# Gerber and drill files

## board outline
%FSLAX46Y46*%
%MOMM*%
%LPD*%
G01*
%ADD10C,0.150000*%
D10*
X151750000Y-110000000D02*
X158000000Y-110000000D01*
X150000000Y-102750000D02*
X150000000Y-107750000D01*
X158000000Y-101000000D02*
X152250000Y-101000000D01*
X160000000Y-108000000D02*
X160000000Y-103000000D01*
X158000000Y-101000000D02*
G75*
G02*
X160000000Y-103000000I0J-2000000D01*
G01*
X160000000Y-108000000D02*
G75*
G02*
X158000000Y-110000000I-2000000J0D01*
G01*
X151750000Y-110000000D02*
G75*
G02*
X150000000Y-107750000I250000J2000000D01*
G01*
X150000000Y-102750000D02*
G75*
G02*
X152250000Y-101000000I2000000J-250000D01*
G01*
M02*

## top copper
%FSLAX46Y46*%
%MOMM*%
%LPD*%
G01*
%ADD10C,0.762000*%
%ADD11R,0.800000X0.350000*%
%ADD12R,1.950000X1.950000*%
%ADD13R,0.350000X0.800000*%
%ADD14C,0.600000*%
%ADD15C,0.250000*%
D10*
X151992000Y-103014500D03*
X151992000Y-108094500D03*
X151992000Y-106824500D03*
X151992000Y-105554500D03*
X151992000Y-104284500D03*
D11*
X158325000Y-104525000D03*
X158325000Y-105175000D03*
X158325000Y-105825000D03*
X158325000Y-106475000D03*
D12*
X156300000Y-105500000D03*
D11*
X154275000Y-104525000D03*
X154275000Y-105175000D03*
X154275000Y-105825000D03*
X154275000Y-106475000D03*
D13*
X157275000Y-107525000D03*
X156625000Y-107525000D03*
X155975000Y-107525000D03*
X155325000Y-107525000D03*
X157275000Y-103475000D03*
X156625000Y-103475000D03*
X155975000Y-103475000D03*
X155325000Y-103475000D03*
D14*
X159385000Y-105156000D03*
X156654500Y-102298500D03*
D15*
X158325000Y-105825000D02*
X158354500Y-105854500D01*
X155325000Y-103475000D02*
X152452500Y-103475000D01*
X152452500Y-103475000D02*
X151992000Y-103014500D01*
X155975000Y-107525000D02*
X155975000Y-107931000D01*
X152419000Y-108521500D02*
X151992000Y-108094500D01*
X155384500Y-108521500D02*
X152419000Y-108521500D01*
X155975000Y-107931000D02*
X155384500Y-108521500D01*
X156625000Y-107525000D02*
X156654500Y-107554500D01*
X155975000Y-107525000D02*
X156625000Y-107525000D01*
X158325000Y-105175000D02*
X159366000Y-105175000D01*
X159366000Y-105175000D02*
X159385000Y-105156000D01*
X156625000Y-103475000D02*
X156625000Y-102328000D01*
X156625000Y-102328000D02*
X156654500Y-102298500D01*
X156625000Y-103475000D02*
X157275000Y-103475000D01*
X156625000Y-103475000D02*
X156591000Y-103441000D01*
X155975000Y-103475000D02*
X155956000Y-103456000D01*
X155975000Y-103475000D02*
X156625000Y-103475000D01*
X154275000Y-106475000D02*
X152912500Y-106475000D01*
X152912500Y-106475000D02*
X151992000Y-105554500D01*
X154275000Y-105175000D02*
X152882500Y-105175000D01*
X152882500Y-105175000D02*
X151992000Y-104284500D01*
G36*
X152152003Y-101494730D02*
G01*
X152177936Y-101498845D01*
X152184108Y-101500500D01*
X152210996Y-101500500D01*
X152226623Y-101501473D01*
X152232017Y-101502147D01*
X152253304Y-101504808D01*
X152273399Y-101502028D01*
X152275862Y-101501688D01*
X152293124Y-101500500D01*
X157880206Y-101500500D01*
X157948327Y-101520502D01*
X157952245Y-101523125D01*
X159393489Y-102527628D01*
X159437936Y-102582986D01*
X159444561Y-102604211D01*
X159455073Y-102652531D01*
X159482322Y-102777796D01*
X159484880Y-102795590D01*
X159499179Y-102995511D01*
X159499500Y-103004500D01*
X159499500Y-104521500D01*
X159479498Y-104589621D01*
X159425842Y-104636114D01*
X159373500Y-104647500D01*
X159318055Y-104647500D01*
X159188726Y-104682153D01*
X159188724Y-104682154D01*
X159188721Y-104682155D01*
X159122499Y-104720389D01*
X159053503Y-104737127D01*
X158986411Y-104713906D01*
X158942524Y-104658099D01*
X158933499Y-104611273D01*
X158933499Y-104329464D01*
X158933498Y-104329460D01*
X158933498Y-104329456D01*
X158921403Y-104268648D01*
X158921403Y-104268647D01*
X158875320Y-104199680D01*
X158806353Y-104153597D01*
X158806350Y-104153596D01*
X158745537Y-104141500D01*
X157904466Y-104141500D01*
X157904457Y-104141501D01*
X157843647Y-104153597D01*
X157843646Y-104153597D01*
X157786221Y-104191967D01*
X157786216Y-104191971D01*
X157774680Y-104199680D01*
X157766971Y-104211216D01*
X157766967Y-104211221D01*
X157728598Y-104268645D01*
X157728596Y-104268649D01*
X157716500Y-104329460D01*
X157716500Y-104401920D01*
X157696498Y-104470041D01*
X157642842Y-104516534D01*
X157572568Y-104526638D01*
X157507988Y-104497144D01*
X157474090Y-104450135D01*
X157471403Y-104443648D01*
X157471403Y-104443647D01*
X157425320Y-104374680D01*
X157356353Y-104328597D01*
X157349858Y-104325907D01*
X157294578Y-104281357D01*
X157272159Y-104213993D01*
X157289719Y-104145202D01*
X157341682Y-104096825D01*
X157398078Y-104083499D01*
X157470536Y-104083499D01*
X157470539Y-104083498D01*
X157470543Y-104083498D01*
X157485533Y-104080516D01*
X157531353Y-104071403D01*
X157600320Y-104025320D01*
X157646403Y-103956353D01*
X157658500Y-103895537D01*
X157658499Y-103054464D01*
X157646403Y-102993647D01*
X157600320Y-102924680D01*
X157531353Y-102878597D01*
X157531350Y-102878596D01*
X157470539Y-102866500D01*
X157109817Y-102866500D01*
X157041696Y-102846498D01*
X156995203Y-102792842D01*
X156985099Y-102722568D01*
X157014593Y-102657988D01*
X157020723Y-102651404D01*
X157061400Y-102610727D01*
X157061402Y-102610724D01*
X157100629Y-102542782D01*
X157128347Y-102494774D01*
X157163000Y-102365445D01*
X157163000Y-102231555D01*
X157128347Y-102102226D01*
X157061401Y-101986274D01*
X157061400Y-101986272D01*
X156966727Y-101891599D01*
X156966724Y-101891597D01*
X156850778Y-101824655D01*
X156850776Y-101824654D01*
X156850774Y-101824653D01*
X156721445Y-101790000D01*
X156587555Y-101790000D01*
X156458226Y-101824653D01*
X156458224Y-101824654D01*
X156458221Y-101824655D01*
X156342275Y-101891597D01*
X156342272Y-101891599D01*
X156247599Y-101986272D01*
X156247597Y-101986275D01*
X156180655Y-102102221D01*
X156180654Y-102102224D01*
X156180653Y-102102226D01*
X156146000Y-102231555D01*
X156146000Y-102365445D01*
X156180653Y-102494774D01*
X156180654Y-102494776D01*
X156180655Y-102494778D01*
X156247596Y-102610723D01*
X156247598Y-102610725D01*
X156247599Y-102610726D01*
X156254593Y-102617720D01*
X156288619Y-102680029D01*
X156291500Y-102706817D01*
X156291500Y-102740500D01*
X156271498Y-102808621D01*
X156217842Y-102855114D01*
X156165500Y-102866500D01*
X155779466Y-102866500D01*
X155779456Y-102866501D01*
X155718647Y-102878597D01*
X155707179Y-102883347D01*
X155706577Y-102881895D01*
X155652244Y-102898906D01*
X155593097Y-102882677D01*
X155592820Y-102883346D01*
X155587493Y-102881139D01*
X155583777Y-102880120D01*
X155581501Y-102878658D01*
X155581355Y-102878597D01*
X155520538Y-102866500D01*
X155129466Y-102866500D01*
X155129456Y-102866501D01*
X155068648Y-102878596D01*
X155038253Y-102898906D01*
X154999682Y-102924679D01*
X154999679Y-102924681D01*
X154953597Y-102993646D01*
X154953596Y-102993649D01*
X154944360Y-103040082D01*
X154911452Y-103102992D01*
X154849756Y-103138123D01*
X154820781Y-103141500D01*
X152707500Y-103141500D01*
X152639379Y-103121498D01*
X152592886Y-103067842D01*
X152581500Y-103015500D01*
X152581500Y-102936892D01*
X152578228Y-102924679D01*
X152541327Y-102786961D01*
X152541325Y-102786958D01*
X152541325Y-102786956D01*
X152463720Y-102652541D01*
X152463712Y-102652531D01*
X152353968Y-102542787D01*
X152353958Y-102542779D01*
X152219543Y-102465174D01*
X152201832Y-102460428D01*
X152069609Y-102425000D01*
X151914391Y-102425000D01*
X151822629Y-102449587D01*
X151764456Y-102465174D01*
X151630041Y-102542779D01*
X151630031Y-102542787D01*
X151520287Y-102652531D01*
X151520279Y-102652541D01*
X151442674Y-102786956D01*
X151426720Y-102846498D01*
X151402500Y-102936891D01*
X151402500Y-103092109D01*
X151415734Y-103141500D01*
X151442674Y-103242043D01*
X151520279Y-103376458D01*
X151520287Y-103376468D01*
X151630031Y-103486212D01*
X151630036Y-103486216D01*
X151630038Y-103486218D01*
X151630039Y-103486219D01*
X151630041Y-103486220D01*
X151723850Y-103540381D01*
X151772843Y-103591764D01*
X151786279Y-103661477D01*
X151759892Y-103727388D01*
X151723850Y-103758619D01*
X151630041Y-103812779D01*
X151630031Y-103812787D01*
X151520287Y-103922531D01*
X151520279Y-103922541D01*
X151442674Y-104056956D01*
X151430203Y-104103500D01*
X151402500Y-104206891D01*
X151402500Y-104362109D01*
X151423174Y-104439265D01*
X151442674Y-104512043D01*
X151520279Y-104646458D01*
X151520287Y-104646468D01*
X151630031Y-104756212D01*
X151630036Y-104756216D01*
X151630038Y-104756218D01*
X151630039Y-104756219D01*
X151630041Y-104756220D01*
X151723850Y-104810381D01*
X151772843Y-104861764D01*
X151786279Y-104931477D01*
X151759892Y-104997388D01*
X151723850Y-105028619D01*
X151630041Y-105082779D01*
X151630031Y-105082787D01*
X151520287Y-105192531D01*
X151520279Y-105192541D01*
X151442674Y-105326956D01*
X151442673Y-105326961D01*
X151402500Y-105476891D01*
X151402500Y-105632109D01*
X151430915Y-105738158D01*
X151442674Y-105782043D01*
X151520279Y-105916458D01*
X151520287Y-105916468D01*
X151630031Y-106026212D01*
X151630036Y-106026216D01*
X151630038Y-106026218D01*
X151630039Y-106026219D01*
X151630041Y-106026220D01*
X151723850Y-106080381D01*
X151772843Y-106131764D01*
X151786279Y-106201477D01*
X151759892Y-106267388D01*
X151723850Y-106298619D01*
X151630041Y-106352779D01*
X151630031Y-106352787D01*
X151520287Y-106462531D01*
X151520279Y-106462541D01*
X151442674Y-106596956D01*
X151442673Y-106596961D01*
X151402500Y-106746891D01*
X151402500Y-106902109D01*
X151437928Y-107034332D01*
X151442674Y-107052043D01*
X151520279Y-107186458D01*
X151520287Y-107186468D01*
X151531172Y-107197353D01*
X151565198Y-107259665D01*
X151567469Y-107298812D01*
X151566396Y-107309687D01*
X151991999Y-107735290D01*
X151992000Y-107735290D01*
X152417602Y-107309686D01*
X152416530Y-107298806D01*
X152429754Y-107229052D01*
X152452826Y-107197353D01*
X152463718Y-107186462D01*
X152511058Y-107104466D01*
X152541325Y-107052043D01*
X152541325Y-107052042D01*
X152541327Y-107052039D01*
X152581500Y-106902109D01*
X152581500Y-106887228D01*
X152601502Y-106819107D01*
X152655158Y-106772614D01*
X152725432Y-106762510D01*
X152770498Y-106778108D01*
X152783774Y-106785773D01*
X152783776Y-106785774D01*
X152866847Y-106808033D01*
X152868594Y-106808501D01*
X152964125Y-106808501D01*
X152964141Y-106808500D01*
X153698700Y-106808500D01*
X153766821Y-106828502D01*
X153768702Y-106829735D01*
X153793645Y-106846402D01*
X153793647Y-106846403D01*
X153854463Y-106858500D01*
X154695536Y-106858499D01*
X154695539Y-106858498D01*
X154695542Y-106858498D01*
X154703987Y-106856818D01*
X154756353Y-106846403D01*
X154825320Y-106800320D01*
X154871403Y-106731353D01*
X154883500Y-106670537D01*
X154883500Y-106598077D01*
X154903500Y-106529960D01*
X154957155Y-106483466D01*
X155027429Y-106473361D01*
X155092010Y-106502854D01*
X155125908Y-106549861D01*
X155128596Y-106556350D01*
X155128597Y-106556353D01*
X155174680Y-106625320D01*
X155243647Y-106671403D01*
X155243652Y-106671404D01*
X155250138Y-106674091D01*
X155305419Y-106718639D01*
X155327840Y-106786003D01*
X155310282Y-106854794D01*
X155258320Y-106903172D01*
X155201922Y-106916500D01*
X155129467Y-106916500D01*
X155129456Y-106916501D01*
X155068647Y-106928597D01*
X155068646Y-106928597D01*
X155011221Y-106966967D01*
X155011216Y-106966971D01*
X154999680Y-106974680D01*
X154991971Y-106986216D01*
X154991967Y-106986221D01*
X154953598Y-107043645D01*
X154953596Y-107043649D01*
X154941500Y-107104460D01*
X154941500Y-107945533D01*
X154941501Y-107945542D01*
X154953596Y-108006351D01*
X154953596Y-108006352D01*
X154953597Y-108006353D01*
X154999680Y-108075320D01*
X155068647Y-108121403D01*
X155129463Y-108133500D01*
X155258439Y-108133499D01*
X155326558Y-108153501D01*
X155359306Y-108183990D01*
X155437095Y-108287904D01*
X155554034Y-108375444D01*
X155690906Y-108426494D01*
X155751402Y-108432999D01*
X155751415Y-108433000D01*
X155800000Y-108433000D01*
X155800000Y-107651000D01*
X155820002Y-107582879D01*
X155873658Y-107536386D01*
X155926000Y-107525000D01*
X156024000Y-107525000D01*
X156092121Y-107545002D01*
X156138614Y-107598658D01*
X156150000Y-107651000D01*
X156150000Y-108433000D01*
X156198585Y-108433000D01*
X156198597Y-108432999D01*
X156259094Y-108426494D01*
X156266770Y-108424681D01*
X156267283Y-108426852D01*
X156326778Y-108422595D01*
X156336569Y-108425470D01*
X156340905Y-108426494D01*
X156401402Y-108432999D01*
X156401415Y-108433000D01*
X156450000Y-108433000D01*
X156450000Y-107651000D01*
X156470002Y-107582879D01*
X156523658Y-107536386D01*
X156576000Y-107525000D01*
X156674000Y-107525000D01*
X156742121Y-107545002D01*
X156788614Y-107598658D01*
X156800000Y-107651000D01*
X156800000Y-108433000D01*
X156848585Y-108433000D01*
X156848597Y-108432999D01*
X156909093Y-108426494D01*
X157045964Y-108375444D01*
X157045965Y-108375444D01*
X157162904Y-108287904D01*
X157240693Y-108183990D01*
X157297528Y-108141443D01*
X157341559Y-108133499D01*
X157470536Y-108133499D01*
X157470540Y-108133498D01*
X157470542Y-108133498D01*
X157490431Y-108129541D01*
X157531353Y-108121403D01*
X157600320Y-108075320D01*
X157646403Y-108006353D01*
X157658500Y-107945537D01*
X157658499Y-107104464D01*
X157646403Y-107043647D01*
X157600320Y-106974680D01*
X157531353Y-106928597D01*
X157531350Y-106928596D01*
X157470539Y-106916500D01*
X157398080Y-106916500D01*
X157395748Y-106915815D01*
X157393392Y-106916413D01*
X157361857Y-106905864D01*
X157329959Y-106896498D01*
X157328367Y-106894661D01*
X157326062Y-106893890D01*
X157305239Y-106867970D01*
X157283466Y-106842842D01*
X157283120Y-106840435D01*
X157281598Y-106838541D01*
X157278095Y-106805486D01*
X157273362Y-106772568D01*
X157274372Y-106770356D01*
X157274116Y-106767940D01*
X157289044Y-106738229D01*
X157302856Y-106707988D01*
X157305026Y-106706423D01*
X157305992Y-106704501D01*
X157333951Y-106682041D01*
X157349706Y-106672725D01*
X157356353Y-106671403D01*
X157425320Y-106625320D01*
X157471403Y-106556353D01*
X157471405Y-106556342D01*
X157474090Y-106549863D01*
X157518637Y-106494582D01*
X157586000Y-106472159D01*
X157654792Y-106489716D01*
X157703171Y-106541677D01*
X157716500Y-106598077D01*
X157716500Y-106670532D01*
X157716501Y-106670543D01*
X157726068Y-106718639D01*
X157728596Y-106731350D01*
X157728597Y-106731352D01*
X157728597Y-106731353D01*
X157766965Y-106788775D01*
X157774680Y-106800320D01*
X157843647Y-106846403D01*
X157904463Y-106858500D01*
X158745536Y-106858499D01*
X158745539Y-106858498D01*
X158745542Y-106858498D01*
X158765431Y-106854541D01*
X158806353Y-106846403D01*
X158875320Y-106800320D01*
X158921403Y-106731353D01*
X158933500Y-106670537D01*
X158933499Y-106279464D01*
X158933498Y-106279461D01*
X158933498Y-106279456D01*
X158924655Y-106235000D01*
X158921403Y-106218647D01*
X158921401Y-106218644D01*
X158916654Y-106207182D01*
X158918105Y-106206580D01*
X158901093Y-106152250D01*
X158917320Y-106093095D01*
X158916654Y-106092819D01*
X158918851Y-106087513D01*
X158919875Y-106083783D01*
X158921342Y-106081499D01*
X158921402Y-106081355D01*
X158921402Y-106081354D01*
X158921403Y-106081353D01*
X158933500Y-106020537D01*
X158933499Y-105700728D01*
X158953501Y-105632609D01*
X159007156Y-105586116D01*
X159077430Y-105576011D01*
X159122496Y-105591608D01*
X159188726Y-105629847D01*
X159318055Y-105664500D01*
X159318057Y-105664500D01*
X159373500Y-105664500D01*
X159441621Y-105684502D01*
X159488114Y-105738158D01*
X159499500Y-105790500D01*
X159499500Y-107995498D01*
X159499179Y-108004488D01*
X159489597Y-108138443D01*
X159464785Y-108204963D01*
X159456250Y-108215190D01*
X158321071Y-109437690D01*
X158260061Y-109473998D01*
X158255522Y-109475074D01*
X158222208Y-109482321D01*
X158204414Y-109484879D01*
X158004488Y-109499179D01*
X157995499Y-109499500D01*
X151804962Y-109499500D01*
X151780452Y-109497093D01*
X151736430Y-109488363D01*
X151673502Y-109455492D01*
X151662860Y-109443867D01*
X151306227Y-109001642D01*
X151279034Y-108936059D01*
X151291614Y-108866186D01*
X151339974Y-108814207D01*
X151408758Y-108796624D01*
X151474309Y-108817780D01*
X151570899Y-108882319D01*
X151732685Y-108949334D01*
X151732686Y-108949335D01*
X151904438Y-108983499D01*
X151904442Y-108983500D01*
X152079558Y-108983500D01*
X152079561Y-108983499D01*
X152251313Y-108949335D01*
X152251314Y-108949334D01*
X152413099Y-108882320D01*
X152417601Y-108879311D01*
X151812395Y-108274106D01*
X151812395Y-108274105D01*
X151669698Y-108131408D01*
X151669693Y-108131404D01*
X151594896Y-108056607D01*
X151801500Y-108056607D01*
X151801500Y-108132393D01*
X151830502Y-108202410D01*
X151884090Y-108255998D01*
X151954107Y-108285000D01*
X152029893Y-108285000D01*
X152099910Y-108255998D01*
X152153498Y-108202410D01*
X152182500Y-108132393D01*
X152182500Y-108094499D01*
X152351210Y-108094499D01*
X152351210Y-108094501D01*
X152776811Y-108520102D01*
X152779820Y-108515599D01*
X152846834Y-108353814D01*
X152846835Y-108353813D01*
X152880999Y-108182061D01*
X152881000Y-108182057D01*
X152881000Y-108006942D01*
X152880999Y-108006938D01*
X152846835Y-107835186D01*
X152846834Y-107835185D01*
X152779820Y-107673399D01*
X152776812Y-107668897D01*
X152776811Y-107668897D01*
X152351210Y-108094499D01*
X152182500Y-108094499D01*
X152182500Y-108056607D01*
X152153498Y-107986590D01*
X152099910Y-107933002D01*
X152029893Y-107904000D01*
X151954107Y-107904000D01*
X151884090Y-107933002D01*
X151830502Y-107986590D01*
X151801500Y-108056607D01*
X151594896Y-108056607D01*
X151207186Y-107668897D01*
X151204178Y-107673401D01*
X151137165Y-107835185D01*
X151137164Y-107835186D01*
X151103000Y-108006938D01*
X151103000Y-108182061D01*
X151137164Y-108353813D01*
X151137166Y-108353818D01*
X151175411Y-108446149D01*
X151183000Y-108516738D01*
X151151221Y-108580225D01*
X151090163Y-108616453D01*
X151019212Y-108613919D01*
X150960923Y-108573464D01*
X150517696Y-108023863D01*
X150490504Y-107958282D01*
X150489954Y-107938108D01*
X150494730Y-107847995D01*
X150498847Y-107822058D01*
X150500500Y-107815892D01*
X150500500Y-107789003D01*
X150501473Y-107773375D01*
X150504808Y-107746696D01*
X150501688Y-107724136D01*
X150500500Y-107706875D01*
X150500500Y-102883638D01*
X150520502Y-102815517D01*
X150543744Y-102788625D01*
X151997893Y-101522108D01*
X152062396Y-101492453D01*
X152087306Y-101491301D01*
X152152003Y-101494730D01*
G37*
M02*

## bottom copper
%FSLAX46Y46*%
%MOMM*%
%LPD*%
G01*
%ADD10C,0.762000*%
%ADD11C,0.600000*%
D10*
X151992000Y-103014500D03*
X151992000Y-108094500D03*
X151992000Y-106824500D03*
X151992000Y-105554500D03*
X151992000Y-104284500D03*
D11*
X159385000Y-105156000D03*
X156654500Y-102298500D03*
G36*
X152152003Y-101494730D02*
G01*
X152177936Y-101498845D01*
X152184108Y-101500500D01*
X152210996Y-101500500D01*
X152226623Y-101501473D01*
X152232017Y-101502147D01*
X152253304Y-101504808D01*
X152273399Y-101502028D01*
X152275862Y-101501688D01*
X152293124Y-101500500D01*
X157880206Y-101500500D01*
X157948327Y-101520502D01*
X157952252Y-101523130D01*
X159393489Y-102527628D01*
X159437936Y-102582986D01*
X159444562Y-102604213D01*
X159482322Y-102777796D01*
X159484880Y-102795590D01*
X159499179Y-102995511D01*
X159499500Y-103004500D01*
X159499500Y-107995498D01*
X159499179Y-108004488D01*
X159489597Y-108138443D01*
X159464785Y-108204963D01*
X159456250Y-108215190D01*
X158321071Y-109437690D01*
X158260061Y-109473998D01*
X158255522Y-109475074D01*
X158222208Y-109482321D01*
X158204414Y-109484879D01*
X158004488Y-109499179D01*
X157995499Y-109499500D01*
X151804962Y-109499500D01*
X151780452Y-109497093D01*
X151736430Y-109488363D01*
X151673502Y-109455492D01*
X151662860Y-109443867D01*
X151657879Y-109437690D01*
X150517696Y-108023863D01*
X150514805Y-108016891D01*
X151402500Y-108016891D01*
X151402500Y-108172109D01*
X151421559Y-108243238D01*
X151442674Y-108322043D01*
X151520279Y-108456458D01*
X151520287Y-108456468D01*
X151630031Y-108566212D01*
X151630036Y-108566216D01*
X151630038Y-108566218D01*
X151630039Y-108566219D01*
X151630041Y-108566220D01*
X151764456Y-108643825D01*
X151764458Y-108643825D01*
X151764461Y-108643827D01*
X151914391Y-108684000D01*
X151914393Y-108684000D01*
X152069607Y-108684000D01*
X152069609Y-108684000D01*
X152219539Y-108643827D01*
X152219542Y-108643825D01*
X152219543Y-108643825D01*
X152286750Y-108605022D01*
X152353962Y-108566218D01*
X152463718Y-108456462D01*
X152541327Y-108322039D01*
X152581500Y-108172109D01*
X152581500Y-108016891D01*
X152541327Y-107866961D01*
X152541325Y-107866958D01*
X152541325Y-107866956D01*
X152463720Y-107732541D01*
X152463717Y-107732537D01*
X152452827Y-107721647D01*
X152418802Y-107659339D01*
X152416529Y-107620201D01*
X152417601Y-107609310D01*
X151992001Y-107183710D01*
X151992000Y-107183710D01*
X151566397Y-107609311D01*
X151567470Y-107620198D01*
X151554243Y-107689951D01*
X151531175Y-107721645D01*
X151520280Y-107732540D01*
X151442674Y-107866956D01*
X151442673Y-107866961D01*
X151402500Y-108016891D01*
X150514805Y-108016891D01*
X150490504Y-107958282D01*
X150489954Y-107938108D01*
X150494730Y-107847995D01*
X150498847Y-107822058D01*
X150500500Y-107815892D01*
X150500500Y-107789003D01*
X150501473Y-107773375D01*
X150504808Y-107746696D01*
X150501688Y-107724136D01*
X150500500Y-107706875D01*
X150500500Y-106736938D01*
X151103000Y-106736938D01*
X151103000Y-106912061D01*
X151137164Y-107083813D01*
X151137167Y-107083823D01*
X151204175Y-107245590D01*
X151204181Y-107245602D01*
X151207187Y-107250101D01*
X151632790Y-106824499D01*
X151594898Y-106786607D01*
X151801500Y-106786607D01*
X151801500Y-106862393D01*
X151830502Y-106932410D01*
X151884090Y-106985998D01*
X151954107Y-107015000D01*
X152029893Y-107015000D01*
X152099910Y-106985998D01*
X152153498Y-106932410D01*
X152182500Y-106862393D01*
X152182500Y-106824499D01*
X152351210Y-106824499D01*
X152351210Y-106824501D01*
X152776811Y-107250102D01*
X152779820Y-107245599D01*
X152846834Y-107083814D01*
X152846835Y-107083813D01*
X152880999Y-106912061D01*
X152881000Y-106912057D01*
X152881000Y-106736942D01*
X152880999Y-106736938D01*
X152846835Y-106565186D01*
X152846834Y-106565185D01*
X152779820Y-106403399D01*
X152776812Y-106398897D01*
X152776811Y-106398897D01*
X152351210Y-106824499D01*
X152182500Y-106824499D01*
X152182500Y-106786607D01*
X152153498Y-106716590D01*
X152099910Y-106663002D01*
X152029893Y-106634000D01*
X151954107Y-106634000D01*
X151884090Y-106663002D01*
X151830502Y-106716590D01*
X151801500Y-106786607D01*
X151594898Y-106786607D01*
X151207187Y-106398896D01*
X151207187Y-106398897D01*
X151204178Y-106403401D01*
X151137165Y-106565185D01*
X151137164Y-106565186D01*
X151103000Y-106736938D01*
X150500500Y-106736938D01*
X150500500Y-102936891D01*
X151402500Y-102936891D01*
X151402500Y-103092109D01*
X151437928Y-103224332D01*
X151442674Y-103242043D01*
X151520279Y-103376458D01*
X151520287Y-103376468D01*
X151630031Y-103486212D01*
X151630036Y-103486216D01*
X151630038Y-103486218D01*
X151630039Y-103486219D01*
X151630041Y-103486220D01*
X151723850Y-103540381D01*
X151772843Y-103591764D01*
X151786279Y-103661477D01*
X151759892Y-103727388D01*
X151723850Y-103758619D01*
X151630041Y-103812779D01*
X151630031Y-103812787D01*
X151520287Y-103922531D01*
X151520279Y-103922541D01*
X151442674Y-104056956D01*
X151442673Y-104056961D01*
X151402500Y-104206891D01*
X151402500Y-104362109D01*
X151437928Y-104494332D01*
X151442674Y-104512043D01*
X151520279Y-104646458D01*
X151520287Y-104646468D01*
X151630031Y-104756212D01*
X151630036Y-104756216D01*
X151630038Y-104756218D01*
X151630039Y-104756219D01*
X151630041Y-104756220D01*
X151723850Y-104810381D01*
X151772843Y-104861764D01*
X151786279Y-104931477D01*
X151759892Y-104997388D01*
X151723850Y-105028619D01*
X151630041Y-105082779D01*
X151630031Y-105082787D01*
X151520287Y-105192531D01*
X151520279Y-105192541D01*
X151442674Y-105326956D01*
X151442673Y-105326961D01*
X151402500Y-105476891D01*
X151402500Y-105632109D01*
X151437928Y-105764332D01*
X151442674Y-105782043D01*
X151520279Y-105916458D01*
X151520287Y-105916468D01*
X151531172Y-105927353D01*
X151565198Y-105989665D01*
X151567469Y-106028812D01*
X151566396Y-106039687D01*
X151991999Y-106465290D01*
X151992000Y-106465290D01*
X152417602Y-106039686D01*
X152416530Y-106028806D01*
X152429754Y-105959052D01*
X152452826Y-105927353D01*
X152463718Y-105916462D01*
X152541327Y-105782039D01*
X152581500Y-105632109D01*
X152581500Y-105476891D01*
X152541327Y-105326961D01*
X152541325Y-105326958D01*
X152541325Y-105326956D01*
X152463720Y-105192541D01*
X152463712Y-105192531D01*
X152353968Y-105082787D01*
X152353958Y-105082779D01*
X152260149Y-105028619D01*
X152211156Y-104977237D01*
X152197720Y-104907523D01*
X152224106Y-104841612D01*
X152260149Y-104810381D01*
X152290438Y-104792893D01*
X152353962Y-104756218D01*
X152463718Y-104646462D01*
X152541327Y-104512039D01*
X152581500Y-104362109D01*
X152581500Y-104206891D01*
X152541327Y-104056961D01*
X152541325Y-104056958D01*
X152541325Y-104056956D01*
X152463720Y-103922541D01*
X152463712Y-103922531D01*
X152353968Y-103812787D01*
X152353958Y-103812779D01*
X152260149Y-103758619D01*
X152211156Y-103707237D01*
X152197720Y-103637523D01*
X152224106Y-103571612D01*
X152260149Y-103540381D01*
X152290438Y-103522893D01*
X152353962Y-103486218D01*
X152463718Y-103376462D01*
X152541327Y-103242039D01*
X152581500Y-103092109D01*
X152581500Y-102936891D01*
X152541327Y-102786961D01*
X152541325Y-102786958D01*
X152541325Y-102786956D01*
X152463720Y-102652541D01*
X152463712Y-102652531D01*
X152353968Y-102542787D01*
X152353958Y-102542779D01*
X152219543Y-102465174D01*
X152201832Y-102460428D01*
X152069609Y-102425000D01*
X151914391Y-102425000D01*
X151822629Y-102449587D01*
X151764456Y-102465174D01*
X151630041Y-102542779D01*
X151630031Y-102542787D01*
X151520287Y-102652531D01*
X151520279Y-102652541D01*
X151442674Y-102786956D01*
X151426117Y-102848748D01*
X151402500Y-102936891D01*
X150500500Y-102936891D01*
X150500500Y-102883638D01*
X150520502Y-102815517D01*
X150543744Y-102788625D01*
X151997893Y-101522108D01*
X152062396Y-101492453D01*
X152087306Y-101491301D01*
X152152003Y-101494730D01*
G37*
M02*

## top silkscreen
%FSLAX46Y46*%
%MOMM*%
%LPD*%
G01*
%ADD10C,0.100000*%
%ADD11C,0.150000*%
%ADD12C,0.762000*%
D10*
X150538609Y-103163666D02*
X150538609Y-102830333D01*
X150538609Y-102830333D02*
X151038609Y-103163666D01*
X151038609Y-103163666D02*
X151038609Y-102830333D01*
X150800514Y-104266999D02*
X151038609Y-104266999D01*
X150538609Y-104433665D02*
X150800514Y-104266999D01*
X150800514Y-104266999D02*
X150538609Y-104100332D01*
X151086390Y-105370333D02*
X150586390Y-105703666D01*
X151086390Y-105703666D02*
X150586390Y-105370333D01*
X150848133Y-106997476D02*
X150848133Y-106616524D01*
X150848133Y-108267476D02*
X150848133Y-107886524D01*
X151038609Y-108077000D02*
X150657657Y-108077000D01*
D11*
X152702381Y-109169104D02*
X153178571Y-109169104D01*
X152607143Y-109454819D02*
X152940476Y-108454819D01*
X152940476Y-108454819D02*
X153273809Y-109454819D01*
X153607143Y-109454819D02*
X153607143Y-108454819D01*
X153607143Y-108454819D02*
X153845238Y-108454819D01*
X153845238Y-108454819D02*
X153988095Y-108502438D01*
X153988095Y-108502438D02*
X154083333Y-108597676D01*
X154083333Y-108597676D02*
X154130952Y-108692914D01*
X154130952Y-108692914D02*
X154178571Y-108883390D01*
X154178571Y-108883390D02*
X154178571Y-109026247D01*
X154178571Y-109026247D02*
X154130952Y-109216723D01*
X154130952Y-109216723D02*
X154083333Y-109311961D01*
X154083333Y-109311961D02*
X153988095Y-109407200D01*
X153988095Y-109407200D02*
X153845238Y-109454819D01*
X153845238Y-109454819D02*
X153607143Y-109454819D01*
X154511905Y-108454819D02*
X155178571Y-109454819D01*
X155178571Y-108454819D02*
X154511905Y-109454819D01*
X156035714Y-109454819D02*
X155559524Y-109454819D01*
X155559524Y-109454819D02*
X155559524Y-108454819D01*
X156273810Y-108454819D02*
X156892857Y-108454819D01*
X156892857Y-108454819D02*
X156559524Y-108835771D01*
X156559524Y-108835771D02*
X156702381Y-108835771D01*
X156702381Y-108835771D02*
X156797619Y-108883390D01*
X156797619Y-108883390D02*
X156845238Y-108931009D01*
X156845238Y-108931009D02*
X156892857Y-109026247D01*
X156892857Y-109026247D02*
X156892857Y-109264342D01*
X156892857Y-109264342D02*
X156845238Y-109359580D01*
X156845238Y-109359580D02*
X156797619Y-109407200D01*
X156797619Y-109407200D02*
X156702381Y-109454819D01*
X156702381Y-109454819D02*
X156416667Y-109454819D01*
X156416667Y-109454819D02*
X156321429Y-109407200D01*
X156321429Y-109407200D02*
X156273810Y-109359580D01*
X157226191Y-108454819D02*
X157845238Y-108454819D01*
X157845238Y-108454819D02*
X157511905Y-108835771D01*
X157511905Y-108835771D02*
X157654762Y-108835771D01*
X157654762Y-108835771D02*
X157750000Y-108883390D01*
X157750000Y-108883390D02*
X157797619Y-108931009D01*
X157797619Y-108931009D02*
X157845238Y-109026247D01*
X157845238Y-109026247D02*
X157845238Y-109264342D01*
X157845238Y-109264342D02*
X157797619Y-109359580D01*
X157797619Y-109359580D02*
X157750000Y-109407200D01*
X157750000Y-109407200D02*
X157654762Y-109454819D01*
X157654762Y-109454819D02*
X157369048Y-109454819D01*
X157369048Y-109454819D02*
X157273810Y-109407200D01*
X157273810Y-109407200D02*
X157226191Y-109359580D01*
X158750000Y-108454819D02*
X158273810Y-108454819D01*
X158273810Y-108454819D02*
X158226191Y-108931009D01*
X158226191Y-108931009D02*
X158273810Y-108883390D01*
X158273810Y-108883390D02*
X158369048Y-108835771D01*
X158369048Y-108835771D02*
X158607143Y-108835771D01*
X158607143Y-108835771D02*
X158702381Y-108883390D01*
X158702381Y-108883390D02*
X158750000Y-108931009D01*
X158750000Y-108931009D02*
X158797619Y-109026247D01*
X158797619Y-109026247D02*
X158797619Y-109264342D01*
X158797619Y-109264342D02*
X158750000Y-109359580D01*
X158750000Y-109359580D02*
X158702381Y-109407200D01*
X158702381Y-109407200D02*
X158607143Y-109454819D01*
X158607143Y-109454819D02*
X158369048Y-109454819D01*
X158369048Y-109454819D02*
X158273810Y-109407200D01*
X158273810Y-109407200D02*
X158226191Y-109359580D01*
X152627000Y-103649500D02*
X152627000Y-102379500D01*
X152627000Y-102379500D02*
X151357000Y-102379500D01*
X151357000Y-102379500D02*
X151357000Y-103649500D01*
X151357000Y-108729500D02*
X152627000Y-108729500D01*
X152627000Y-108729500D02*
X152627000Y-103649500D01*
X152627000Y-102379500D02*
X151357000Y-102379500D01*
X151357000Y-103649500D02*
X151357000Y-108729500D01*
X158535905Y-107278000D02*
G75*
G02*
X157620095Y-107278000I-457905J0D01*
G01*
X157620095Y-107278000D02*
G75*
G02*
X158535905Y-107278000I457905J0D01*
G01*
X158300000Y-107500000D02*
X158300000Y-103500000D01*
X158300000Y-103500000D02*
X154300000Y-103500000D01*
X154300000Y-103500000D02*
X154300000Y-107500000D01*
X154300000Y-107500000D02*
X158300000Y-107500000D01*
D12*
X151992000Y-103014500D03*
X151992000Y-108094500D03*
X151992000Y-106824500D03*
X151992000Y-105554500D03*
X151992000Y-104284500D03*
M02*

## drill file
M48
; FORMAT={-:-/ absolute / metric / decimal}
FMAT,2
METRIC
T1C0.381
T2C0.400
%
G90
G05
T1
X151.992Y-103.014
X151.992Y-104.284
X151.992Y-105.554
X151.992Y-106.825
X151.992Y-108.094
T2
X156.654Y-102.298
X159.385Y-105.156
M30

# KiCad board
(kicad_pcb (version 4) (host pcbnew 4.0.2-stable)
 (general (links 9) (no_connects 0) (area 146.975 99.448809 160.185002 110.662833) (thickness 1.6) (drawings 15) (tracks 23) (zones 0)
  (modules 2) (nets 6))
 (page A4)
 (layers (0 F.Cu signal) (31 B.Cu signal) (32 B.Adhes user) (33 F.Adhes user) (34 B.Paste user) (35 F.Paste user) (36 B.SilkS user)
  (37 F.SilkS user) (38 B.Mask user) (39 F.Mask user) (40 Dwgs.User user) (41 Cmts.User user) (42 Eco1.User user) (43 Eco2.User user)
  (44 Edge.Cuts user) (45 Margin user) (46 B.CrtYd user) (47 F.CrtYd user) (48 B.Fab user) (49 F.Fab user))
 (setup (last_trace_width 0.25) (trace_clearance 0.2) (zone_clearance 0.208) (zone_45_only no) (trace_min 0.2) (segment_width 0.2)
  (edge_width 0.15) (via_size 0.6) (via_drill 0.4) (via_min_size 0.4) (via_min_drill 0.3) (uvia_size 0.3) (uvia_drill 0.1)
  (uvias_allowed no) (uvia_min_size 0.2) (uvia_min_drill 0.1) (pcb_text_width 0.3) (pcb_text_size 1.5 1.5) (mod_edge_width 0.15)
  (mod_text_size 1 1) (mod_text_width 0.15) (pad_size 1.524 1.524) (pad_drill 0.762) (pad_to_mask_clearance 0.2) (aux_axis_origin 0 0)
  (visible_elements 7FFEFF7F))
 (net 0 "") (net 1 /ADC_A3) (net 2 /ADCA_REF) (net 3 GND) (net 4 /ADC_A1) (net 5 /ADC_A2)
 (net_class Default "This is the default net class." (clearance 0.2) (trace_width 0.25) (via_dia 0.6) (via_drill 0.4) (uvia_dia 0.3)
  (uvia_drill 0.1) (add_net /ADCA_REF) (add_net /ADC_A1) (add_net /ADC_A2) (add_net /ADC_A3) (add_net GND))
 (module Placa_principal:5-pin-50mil (layer F.Cu) (at 151.992 105.5545 90)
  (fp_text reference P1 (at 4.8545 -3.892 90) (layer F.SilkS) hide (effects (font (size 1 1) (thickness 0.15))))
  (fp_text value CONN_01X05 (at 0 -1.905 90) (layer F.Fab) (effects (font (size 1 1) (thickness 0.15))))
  (fp_line (start 1.905 0.635) (end 3.175 0.635) (layer F.SilkS) (width 0.15))
  (fp_line (start 3.175 0.635) (end 3.175 -0.635) (layer F.SilkS) (width 0.15))
  (fp_line (start 3.175 -0.635) (end 1.905 -0.635) (layer F.SilkS) (width 0.15))
  (fp_line (start -3.175 -0.635) (end -3.175 0.635) (layer F.SilkS) (width 0.15))
  (fp_line (start -3.175 0.635) (end 1.905 0.635) (layer F.SilkS) (width 0.15))
  (fp_line (start 3.175 0.635) (end 3.175 -0.635) (layer F.SilkS) (width 0.15))
  (fp_line (start 1.905 -0.635) (end -3.175 -0.635) (layer F.SilkS) (width 0.15))
  (pad 5 thru_hole circle (at 2.54 0 90) (size 0.762 0.762) (drill 0.381) (layers *.Cu *.Mask F.SilkS) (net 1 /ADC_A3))
  (pad 1 thru_hole circle (at -2.54 0 90) (size 0.762 0.762) (drill 0.381) (layers *.Cu *.Mask F.SilkS) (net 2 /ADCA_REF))
  (pad 2 thru_hole circle (at -1.27 0 90) (size 0.762 0.762) (drill 0.381) (layers *.Cu *.Mask F.SilkS) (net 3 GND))
  (pad 3 thru_hole circle (at 0 0 90) (size 0.762 0.762) (drill 0.381) (layers *.Cu *.Mask F.SilkS) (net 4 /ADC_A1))
  (pad 4 thru_hole circle (at 1.27 0 90) (size 0.762 0.762) (drill 0.381) (layers *.Cu *.Mask F.SilkS) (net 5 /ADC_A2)))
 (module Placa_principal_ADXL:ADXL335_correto (layer F.Cu) (at 156.3 105.5 180)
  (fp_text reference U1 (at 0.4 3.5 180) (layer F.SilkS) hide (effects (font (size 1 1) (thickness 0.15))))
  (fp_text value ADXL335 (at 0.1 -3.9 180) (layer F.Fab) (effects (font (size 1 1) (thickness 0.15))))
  (fp_circle (center -1.778 -1.778) (end -1.397 -1.524) (layer F.SilkS) (width 0.15))
  (fp_line (start -2 -2) (end -2 2) (layer F.SilkS) (width 0.15))
  (fp_line (start -2 2) (end 2 2) (layer F.SilkS) (width 0.15))
  (fp_line (start 2 2) (end 2 -2) (layer F.SilkS) (width 0.15))
  (fp_line (start 2 -2) (end -2 -2) (layer F.SilkS) (width 0.15))
  (pad 4 smd rect (at -2.025 0.975 180) (size 0.8 0.35) (layers F.Cu F.Paste F.Mask))
  (pad 3 smd rect (at -2.025 0.325 180) (size 0.8 0.35) (layers F.Cu F.Paste F.Mask) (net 3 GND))
  (pad 2 smd rect (at -2.025 -0.325 180) (size 0.8 0.35) (layers F.Cu F.Paste F.Mask))
  (pad 1 smd rect (at -2.025 -0.975 180) (size 0.8 0.35) (layers F.Cu F.Paste F.Mask))
  (pad ~ smd rect (at 0 0 180) (size 1.95 1.95) (layers F.Cu F.Paste F.Mask))
  (pad 9 smd rect (at 2.025 0.975 180) (size 0.8 0.35) (layers F.Cu F.Paste F.Mask))
  (pad 10 smd rect (at 2.025 0.325 180) (size 0.8 0.35) (layers F.Cu F.Paste F.Mask) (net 5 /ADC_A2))
  (pad 11 smd rect (at 2.025 -0.325 180) (size 0.8 0.35) (layers F.Cu F.Paste F.Mask))
  (pad 12 smd rect (at 2.025 -0.975 180) (size 0.8 0.35) (layers F.Cu F.Paste F.Mask) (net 4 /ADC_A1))
  (pad 16 smd rect (at -0.975 -2.025 180) (size 0.35 0.8) (layers F.Cu F.Paste F.Mask))
  (pad 15 smd rect (at -0.325 -2.025 180) (size 0.35 0.8) (layers F.Cu F.Paste F.Mask) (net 2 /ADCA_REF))
  (pad 14 smd rect (at 0.325 -2.025 180) (size 0.35 0.8) (layers F.Cu F.Paste F.Mask) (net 2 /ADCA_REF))
  (pad 13 smd rect (at 0.975 -2.025 180) (size 0.35 0.8) (layers F.Cu F.Paste F.Mask))
  (pad 5 smd rect (at -0.975 2.025 180) (size 0.35 0.8) (layers F.Cu F.Paste F.Mask) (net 3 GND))
  (pad 6 smd rect (at -0.325 2.025 180) (size 0.35 0.8) (layers F.Cu F.Paste F.Mask) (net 3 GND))
  (pad 7 smd rect (at 0.325 2.025 180) (size 0.35 0.8) (layers F.Cu F.Paste F.Mask) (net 3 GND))
  (pad 8 smd rect (at 0.975 2.025 180) (size 0.35 0.8) (layers F.Cu F.Paste F.Mask) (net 1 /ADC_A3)))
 (gr_line (start 151.75 110) (end 158 110) (angle 90) (layer Edge.Cuts) (width 0.15))
 (gr_line (start 150 102.75) (end 150 107.75) (angle 90) (layer Edge.Cuts) (width 0.15))
 (gr_line (start 158 101) (end 152.25 101) (angle 90) (layer Edge.Cuts) (width 0.15))
 (gr_line (start 160 108) (end 160 103) (angle 90) (layer Edge.Cuts) (width 0.15))
 (gr_arc (start 158 103) (end 158 101) (angle 90) (layer Edge.Cuts) (width 0.15))
 (gr_arc (start 158 108) (end 160 108) (angle 90) (layer Edge.Cuts) (width 0.15))
 (gr_arc (start 152 108) (end 151.75 110) (angle 90) (layer Edge.Cuts) (width 0.15))
 (gr_arc (start 152 103) (end 150 102.75) (angle 90) (layer Edge.Cuts) (width 0.15))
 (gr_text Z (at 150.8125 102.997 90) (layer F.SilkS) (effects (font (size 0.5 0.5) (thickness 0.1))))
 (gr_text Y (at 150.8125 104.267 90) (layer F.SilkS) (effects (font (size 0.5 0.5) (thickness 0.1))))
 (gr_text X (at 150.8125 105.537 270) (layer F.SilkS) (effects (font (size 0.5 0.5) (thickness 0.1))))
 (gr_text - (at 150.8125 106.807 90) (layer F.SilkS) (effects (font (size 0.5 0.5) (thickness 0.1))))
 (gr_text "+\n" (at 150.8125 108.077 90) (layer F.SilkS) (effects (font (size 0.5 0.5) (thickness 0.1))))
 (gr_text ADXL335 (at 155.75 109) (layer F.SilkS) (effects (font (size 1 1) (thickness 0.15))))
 (segment (start 158.325 105.825) (end 158.3545 105.8545) (width 0.25) (layer F.Cu) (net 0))
 (segment (start 155.325 103.475) (end 152.4525 103.475) (width 0.25) (layer F.Cu) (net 1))
 (segment (start 152.4525 103.475) (end 151.992 103.0145) (width 0.25) (layer F.Cu) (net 1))
 (segment (start 155.975 107.525) (end 155.975 107.931) (width 0.25) (layer F.Cu) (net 2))
 (segment (start 152.419 108.5215) (end 151.992 108.0945) (width 0.25) (layer F.Cu) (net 2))
 (segment (start 155.3845 108.5215) (end 152.419 108.5215) (width 0.25) (layer F.Cu) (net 2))
 (segment (start 155.975 107.931) (end 155.3845 108.5215) (width 0.25) (layer F.Cu) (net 2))
 (segment (start 156.625 107.525) (end 156.6545 107.5545) (width 0.25) (layer F.Cu) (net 2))
 (segment (start 155.975 107.525) (end 156.625 107.525) (width 0.25) (layer F.Cu) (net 2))
 (segment (start 158.325 105.175) (end 159.366 105.175) (width 0.25) (layer F.Cu) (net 3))
 (via (at 159.385 105.156) (size 0.6) (drill 0.4) (layers F.Cu B.Cu) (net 3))
 (segment (start 159.366 105.175) (end 159.385 105.156) (width 0.25) (layer F.Cu) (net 3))
 (segment (start 156.625 103.475) (end 156.625 102.328) (width 0.25) (layer F.Cu) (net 3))
 (via (at 156.6545 102.2985) (size 0.6) (drill 0.4) (layers F.Cu B.Cu) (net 3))
 (segment (start 156.625 102.328) (end 156.6545 102.2985) (width 0.25) (layer F.Cu) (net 3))
 (segment (start 156.625 103.475) (end 157.275 103.475) (width 0.25) (layer F.Cu) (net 3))
 (segment (start 156.625 103.475) (end 156.591 103.441) (width 0.25) (layer F.Cu) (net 3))
 (segment (start 155.975 103.475) (end 155.956 103.456) (width 0.25) (layer F.Cu) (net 3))
 (segment (start 155.975 103.475) (end 156.625 103.475) (width 0.25) (layer F.Cu) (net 3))
 (segment (start 154.275 106.475) (end 152.9125 106.475) (width 0.25) (layer F.Cu) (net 4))
 (segment (start 152.9125 106.475) (end 151.992 105.5545) (width 0.25) (layer F.Cu) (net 4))
 (segment (start 154.275 105.175) (end 152.8825 105.175) (width 0.25) (layer F.Cu) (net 5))
 (segment (start 152.8825 105.175) (end 151.992 104.2845) (width 0.25) (layer F.Cu) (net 5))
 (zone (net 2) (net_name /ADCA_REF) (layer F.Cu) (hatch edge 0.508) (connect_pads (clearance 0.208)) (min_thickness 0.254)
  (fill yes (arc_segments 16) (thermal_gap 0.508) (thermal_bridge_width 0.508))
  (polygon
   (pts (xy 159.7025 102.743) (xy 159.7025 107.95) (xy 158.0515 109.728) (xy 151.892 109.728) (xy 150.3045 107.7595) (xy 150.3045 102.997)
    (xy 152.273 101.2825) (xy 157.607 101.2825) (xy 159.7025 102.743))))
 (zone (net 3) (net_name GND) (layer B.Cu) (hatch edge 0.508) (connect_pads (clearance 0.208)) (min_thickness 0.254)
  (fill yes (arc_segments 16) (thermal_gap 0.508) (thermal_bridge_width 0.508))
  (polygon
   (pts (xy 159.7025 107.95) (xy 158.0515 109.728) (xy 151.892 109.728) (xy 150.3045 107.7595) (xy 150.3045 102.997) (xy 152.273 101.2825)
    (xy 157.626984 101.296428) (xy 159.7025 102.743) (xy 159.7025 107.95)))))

